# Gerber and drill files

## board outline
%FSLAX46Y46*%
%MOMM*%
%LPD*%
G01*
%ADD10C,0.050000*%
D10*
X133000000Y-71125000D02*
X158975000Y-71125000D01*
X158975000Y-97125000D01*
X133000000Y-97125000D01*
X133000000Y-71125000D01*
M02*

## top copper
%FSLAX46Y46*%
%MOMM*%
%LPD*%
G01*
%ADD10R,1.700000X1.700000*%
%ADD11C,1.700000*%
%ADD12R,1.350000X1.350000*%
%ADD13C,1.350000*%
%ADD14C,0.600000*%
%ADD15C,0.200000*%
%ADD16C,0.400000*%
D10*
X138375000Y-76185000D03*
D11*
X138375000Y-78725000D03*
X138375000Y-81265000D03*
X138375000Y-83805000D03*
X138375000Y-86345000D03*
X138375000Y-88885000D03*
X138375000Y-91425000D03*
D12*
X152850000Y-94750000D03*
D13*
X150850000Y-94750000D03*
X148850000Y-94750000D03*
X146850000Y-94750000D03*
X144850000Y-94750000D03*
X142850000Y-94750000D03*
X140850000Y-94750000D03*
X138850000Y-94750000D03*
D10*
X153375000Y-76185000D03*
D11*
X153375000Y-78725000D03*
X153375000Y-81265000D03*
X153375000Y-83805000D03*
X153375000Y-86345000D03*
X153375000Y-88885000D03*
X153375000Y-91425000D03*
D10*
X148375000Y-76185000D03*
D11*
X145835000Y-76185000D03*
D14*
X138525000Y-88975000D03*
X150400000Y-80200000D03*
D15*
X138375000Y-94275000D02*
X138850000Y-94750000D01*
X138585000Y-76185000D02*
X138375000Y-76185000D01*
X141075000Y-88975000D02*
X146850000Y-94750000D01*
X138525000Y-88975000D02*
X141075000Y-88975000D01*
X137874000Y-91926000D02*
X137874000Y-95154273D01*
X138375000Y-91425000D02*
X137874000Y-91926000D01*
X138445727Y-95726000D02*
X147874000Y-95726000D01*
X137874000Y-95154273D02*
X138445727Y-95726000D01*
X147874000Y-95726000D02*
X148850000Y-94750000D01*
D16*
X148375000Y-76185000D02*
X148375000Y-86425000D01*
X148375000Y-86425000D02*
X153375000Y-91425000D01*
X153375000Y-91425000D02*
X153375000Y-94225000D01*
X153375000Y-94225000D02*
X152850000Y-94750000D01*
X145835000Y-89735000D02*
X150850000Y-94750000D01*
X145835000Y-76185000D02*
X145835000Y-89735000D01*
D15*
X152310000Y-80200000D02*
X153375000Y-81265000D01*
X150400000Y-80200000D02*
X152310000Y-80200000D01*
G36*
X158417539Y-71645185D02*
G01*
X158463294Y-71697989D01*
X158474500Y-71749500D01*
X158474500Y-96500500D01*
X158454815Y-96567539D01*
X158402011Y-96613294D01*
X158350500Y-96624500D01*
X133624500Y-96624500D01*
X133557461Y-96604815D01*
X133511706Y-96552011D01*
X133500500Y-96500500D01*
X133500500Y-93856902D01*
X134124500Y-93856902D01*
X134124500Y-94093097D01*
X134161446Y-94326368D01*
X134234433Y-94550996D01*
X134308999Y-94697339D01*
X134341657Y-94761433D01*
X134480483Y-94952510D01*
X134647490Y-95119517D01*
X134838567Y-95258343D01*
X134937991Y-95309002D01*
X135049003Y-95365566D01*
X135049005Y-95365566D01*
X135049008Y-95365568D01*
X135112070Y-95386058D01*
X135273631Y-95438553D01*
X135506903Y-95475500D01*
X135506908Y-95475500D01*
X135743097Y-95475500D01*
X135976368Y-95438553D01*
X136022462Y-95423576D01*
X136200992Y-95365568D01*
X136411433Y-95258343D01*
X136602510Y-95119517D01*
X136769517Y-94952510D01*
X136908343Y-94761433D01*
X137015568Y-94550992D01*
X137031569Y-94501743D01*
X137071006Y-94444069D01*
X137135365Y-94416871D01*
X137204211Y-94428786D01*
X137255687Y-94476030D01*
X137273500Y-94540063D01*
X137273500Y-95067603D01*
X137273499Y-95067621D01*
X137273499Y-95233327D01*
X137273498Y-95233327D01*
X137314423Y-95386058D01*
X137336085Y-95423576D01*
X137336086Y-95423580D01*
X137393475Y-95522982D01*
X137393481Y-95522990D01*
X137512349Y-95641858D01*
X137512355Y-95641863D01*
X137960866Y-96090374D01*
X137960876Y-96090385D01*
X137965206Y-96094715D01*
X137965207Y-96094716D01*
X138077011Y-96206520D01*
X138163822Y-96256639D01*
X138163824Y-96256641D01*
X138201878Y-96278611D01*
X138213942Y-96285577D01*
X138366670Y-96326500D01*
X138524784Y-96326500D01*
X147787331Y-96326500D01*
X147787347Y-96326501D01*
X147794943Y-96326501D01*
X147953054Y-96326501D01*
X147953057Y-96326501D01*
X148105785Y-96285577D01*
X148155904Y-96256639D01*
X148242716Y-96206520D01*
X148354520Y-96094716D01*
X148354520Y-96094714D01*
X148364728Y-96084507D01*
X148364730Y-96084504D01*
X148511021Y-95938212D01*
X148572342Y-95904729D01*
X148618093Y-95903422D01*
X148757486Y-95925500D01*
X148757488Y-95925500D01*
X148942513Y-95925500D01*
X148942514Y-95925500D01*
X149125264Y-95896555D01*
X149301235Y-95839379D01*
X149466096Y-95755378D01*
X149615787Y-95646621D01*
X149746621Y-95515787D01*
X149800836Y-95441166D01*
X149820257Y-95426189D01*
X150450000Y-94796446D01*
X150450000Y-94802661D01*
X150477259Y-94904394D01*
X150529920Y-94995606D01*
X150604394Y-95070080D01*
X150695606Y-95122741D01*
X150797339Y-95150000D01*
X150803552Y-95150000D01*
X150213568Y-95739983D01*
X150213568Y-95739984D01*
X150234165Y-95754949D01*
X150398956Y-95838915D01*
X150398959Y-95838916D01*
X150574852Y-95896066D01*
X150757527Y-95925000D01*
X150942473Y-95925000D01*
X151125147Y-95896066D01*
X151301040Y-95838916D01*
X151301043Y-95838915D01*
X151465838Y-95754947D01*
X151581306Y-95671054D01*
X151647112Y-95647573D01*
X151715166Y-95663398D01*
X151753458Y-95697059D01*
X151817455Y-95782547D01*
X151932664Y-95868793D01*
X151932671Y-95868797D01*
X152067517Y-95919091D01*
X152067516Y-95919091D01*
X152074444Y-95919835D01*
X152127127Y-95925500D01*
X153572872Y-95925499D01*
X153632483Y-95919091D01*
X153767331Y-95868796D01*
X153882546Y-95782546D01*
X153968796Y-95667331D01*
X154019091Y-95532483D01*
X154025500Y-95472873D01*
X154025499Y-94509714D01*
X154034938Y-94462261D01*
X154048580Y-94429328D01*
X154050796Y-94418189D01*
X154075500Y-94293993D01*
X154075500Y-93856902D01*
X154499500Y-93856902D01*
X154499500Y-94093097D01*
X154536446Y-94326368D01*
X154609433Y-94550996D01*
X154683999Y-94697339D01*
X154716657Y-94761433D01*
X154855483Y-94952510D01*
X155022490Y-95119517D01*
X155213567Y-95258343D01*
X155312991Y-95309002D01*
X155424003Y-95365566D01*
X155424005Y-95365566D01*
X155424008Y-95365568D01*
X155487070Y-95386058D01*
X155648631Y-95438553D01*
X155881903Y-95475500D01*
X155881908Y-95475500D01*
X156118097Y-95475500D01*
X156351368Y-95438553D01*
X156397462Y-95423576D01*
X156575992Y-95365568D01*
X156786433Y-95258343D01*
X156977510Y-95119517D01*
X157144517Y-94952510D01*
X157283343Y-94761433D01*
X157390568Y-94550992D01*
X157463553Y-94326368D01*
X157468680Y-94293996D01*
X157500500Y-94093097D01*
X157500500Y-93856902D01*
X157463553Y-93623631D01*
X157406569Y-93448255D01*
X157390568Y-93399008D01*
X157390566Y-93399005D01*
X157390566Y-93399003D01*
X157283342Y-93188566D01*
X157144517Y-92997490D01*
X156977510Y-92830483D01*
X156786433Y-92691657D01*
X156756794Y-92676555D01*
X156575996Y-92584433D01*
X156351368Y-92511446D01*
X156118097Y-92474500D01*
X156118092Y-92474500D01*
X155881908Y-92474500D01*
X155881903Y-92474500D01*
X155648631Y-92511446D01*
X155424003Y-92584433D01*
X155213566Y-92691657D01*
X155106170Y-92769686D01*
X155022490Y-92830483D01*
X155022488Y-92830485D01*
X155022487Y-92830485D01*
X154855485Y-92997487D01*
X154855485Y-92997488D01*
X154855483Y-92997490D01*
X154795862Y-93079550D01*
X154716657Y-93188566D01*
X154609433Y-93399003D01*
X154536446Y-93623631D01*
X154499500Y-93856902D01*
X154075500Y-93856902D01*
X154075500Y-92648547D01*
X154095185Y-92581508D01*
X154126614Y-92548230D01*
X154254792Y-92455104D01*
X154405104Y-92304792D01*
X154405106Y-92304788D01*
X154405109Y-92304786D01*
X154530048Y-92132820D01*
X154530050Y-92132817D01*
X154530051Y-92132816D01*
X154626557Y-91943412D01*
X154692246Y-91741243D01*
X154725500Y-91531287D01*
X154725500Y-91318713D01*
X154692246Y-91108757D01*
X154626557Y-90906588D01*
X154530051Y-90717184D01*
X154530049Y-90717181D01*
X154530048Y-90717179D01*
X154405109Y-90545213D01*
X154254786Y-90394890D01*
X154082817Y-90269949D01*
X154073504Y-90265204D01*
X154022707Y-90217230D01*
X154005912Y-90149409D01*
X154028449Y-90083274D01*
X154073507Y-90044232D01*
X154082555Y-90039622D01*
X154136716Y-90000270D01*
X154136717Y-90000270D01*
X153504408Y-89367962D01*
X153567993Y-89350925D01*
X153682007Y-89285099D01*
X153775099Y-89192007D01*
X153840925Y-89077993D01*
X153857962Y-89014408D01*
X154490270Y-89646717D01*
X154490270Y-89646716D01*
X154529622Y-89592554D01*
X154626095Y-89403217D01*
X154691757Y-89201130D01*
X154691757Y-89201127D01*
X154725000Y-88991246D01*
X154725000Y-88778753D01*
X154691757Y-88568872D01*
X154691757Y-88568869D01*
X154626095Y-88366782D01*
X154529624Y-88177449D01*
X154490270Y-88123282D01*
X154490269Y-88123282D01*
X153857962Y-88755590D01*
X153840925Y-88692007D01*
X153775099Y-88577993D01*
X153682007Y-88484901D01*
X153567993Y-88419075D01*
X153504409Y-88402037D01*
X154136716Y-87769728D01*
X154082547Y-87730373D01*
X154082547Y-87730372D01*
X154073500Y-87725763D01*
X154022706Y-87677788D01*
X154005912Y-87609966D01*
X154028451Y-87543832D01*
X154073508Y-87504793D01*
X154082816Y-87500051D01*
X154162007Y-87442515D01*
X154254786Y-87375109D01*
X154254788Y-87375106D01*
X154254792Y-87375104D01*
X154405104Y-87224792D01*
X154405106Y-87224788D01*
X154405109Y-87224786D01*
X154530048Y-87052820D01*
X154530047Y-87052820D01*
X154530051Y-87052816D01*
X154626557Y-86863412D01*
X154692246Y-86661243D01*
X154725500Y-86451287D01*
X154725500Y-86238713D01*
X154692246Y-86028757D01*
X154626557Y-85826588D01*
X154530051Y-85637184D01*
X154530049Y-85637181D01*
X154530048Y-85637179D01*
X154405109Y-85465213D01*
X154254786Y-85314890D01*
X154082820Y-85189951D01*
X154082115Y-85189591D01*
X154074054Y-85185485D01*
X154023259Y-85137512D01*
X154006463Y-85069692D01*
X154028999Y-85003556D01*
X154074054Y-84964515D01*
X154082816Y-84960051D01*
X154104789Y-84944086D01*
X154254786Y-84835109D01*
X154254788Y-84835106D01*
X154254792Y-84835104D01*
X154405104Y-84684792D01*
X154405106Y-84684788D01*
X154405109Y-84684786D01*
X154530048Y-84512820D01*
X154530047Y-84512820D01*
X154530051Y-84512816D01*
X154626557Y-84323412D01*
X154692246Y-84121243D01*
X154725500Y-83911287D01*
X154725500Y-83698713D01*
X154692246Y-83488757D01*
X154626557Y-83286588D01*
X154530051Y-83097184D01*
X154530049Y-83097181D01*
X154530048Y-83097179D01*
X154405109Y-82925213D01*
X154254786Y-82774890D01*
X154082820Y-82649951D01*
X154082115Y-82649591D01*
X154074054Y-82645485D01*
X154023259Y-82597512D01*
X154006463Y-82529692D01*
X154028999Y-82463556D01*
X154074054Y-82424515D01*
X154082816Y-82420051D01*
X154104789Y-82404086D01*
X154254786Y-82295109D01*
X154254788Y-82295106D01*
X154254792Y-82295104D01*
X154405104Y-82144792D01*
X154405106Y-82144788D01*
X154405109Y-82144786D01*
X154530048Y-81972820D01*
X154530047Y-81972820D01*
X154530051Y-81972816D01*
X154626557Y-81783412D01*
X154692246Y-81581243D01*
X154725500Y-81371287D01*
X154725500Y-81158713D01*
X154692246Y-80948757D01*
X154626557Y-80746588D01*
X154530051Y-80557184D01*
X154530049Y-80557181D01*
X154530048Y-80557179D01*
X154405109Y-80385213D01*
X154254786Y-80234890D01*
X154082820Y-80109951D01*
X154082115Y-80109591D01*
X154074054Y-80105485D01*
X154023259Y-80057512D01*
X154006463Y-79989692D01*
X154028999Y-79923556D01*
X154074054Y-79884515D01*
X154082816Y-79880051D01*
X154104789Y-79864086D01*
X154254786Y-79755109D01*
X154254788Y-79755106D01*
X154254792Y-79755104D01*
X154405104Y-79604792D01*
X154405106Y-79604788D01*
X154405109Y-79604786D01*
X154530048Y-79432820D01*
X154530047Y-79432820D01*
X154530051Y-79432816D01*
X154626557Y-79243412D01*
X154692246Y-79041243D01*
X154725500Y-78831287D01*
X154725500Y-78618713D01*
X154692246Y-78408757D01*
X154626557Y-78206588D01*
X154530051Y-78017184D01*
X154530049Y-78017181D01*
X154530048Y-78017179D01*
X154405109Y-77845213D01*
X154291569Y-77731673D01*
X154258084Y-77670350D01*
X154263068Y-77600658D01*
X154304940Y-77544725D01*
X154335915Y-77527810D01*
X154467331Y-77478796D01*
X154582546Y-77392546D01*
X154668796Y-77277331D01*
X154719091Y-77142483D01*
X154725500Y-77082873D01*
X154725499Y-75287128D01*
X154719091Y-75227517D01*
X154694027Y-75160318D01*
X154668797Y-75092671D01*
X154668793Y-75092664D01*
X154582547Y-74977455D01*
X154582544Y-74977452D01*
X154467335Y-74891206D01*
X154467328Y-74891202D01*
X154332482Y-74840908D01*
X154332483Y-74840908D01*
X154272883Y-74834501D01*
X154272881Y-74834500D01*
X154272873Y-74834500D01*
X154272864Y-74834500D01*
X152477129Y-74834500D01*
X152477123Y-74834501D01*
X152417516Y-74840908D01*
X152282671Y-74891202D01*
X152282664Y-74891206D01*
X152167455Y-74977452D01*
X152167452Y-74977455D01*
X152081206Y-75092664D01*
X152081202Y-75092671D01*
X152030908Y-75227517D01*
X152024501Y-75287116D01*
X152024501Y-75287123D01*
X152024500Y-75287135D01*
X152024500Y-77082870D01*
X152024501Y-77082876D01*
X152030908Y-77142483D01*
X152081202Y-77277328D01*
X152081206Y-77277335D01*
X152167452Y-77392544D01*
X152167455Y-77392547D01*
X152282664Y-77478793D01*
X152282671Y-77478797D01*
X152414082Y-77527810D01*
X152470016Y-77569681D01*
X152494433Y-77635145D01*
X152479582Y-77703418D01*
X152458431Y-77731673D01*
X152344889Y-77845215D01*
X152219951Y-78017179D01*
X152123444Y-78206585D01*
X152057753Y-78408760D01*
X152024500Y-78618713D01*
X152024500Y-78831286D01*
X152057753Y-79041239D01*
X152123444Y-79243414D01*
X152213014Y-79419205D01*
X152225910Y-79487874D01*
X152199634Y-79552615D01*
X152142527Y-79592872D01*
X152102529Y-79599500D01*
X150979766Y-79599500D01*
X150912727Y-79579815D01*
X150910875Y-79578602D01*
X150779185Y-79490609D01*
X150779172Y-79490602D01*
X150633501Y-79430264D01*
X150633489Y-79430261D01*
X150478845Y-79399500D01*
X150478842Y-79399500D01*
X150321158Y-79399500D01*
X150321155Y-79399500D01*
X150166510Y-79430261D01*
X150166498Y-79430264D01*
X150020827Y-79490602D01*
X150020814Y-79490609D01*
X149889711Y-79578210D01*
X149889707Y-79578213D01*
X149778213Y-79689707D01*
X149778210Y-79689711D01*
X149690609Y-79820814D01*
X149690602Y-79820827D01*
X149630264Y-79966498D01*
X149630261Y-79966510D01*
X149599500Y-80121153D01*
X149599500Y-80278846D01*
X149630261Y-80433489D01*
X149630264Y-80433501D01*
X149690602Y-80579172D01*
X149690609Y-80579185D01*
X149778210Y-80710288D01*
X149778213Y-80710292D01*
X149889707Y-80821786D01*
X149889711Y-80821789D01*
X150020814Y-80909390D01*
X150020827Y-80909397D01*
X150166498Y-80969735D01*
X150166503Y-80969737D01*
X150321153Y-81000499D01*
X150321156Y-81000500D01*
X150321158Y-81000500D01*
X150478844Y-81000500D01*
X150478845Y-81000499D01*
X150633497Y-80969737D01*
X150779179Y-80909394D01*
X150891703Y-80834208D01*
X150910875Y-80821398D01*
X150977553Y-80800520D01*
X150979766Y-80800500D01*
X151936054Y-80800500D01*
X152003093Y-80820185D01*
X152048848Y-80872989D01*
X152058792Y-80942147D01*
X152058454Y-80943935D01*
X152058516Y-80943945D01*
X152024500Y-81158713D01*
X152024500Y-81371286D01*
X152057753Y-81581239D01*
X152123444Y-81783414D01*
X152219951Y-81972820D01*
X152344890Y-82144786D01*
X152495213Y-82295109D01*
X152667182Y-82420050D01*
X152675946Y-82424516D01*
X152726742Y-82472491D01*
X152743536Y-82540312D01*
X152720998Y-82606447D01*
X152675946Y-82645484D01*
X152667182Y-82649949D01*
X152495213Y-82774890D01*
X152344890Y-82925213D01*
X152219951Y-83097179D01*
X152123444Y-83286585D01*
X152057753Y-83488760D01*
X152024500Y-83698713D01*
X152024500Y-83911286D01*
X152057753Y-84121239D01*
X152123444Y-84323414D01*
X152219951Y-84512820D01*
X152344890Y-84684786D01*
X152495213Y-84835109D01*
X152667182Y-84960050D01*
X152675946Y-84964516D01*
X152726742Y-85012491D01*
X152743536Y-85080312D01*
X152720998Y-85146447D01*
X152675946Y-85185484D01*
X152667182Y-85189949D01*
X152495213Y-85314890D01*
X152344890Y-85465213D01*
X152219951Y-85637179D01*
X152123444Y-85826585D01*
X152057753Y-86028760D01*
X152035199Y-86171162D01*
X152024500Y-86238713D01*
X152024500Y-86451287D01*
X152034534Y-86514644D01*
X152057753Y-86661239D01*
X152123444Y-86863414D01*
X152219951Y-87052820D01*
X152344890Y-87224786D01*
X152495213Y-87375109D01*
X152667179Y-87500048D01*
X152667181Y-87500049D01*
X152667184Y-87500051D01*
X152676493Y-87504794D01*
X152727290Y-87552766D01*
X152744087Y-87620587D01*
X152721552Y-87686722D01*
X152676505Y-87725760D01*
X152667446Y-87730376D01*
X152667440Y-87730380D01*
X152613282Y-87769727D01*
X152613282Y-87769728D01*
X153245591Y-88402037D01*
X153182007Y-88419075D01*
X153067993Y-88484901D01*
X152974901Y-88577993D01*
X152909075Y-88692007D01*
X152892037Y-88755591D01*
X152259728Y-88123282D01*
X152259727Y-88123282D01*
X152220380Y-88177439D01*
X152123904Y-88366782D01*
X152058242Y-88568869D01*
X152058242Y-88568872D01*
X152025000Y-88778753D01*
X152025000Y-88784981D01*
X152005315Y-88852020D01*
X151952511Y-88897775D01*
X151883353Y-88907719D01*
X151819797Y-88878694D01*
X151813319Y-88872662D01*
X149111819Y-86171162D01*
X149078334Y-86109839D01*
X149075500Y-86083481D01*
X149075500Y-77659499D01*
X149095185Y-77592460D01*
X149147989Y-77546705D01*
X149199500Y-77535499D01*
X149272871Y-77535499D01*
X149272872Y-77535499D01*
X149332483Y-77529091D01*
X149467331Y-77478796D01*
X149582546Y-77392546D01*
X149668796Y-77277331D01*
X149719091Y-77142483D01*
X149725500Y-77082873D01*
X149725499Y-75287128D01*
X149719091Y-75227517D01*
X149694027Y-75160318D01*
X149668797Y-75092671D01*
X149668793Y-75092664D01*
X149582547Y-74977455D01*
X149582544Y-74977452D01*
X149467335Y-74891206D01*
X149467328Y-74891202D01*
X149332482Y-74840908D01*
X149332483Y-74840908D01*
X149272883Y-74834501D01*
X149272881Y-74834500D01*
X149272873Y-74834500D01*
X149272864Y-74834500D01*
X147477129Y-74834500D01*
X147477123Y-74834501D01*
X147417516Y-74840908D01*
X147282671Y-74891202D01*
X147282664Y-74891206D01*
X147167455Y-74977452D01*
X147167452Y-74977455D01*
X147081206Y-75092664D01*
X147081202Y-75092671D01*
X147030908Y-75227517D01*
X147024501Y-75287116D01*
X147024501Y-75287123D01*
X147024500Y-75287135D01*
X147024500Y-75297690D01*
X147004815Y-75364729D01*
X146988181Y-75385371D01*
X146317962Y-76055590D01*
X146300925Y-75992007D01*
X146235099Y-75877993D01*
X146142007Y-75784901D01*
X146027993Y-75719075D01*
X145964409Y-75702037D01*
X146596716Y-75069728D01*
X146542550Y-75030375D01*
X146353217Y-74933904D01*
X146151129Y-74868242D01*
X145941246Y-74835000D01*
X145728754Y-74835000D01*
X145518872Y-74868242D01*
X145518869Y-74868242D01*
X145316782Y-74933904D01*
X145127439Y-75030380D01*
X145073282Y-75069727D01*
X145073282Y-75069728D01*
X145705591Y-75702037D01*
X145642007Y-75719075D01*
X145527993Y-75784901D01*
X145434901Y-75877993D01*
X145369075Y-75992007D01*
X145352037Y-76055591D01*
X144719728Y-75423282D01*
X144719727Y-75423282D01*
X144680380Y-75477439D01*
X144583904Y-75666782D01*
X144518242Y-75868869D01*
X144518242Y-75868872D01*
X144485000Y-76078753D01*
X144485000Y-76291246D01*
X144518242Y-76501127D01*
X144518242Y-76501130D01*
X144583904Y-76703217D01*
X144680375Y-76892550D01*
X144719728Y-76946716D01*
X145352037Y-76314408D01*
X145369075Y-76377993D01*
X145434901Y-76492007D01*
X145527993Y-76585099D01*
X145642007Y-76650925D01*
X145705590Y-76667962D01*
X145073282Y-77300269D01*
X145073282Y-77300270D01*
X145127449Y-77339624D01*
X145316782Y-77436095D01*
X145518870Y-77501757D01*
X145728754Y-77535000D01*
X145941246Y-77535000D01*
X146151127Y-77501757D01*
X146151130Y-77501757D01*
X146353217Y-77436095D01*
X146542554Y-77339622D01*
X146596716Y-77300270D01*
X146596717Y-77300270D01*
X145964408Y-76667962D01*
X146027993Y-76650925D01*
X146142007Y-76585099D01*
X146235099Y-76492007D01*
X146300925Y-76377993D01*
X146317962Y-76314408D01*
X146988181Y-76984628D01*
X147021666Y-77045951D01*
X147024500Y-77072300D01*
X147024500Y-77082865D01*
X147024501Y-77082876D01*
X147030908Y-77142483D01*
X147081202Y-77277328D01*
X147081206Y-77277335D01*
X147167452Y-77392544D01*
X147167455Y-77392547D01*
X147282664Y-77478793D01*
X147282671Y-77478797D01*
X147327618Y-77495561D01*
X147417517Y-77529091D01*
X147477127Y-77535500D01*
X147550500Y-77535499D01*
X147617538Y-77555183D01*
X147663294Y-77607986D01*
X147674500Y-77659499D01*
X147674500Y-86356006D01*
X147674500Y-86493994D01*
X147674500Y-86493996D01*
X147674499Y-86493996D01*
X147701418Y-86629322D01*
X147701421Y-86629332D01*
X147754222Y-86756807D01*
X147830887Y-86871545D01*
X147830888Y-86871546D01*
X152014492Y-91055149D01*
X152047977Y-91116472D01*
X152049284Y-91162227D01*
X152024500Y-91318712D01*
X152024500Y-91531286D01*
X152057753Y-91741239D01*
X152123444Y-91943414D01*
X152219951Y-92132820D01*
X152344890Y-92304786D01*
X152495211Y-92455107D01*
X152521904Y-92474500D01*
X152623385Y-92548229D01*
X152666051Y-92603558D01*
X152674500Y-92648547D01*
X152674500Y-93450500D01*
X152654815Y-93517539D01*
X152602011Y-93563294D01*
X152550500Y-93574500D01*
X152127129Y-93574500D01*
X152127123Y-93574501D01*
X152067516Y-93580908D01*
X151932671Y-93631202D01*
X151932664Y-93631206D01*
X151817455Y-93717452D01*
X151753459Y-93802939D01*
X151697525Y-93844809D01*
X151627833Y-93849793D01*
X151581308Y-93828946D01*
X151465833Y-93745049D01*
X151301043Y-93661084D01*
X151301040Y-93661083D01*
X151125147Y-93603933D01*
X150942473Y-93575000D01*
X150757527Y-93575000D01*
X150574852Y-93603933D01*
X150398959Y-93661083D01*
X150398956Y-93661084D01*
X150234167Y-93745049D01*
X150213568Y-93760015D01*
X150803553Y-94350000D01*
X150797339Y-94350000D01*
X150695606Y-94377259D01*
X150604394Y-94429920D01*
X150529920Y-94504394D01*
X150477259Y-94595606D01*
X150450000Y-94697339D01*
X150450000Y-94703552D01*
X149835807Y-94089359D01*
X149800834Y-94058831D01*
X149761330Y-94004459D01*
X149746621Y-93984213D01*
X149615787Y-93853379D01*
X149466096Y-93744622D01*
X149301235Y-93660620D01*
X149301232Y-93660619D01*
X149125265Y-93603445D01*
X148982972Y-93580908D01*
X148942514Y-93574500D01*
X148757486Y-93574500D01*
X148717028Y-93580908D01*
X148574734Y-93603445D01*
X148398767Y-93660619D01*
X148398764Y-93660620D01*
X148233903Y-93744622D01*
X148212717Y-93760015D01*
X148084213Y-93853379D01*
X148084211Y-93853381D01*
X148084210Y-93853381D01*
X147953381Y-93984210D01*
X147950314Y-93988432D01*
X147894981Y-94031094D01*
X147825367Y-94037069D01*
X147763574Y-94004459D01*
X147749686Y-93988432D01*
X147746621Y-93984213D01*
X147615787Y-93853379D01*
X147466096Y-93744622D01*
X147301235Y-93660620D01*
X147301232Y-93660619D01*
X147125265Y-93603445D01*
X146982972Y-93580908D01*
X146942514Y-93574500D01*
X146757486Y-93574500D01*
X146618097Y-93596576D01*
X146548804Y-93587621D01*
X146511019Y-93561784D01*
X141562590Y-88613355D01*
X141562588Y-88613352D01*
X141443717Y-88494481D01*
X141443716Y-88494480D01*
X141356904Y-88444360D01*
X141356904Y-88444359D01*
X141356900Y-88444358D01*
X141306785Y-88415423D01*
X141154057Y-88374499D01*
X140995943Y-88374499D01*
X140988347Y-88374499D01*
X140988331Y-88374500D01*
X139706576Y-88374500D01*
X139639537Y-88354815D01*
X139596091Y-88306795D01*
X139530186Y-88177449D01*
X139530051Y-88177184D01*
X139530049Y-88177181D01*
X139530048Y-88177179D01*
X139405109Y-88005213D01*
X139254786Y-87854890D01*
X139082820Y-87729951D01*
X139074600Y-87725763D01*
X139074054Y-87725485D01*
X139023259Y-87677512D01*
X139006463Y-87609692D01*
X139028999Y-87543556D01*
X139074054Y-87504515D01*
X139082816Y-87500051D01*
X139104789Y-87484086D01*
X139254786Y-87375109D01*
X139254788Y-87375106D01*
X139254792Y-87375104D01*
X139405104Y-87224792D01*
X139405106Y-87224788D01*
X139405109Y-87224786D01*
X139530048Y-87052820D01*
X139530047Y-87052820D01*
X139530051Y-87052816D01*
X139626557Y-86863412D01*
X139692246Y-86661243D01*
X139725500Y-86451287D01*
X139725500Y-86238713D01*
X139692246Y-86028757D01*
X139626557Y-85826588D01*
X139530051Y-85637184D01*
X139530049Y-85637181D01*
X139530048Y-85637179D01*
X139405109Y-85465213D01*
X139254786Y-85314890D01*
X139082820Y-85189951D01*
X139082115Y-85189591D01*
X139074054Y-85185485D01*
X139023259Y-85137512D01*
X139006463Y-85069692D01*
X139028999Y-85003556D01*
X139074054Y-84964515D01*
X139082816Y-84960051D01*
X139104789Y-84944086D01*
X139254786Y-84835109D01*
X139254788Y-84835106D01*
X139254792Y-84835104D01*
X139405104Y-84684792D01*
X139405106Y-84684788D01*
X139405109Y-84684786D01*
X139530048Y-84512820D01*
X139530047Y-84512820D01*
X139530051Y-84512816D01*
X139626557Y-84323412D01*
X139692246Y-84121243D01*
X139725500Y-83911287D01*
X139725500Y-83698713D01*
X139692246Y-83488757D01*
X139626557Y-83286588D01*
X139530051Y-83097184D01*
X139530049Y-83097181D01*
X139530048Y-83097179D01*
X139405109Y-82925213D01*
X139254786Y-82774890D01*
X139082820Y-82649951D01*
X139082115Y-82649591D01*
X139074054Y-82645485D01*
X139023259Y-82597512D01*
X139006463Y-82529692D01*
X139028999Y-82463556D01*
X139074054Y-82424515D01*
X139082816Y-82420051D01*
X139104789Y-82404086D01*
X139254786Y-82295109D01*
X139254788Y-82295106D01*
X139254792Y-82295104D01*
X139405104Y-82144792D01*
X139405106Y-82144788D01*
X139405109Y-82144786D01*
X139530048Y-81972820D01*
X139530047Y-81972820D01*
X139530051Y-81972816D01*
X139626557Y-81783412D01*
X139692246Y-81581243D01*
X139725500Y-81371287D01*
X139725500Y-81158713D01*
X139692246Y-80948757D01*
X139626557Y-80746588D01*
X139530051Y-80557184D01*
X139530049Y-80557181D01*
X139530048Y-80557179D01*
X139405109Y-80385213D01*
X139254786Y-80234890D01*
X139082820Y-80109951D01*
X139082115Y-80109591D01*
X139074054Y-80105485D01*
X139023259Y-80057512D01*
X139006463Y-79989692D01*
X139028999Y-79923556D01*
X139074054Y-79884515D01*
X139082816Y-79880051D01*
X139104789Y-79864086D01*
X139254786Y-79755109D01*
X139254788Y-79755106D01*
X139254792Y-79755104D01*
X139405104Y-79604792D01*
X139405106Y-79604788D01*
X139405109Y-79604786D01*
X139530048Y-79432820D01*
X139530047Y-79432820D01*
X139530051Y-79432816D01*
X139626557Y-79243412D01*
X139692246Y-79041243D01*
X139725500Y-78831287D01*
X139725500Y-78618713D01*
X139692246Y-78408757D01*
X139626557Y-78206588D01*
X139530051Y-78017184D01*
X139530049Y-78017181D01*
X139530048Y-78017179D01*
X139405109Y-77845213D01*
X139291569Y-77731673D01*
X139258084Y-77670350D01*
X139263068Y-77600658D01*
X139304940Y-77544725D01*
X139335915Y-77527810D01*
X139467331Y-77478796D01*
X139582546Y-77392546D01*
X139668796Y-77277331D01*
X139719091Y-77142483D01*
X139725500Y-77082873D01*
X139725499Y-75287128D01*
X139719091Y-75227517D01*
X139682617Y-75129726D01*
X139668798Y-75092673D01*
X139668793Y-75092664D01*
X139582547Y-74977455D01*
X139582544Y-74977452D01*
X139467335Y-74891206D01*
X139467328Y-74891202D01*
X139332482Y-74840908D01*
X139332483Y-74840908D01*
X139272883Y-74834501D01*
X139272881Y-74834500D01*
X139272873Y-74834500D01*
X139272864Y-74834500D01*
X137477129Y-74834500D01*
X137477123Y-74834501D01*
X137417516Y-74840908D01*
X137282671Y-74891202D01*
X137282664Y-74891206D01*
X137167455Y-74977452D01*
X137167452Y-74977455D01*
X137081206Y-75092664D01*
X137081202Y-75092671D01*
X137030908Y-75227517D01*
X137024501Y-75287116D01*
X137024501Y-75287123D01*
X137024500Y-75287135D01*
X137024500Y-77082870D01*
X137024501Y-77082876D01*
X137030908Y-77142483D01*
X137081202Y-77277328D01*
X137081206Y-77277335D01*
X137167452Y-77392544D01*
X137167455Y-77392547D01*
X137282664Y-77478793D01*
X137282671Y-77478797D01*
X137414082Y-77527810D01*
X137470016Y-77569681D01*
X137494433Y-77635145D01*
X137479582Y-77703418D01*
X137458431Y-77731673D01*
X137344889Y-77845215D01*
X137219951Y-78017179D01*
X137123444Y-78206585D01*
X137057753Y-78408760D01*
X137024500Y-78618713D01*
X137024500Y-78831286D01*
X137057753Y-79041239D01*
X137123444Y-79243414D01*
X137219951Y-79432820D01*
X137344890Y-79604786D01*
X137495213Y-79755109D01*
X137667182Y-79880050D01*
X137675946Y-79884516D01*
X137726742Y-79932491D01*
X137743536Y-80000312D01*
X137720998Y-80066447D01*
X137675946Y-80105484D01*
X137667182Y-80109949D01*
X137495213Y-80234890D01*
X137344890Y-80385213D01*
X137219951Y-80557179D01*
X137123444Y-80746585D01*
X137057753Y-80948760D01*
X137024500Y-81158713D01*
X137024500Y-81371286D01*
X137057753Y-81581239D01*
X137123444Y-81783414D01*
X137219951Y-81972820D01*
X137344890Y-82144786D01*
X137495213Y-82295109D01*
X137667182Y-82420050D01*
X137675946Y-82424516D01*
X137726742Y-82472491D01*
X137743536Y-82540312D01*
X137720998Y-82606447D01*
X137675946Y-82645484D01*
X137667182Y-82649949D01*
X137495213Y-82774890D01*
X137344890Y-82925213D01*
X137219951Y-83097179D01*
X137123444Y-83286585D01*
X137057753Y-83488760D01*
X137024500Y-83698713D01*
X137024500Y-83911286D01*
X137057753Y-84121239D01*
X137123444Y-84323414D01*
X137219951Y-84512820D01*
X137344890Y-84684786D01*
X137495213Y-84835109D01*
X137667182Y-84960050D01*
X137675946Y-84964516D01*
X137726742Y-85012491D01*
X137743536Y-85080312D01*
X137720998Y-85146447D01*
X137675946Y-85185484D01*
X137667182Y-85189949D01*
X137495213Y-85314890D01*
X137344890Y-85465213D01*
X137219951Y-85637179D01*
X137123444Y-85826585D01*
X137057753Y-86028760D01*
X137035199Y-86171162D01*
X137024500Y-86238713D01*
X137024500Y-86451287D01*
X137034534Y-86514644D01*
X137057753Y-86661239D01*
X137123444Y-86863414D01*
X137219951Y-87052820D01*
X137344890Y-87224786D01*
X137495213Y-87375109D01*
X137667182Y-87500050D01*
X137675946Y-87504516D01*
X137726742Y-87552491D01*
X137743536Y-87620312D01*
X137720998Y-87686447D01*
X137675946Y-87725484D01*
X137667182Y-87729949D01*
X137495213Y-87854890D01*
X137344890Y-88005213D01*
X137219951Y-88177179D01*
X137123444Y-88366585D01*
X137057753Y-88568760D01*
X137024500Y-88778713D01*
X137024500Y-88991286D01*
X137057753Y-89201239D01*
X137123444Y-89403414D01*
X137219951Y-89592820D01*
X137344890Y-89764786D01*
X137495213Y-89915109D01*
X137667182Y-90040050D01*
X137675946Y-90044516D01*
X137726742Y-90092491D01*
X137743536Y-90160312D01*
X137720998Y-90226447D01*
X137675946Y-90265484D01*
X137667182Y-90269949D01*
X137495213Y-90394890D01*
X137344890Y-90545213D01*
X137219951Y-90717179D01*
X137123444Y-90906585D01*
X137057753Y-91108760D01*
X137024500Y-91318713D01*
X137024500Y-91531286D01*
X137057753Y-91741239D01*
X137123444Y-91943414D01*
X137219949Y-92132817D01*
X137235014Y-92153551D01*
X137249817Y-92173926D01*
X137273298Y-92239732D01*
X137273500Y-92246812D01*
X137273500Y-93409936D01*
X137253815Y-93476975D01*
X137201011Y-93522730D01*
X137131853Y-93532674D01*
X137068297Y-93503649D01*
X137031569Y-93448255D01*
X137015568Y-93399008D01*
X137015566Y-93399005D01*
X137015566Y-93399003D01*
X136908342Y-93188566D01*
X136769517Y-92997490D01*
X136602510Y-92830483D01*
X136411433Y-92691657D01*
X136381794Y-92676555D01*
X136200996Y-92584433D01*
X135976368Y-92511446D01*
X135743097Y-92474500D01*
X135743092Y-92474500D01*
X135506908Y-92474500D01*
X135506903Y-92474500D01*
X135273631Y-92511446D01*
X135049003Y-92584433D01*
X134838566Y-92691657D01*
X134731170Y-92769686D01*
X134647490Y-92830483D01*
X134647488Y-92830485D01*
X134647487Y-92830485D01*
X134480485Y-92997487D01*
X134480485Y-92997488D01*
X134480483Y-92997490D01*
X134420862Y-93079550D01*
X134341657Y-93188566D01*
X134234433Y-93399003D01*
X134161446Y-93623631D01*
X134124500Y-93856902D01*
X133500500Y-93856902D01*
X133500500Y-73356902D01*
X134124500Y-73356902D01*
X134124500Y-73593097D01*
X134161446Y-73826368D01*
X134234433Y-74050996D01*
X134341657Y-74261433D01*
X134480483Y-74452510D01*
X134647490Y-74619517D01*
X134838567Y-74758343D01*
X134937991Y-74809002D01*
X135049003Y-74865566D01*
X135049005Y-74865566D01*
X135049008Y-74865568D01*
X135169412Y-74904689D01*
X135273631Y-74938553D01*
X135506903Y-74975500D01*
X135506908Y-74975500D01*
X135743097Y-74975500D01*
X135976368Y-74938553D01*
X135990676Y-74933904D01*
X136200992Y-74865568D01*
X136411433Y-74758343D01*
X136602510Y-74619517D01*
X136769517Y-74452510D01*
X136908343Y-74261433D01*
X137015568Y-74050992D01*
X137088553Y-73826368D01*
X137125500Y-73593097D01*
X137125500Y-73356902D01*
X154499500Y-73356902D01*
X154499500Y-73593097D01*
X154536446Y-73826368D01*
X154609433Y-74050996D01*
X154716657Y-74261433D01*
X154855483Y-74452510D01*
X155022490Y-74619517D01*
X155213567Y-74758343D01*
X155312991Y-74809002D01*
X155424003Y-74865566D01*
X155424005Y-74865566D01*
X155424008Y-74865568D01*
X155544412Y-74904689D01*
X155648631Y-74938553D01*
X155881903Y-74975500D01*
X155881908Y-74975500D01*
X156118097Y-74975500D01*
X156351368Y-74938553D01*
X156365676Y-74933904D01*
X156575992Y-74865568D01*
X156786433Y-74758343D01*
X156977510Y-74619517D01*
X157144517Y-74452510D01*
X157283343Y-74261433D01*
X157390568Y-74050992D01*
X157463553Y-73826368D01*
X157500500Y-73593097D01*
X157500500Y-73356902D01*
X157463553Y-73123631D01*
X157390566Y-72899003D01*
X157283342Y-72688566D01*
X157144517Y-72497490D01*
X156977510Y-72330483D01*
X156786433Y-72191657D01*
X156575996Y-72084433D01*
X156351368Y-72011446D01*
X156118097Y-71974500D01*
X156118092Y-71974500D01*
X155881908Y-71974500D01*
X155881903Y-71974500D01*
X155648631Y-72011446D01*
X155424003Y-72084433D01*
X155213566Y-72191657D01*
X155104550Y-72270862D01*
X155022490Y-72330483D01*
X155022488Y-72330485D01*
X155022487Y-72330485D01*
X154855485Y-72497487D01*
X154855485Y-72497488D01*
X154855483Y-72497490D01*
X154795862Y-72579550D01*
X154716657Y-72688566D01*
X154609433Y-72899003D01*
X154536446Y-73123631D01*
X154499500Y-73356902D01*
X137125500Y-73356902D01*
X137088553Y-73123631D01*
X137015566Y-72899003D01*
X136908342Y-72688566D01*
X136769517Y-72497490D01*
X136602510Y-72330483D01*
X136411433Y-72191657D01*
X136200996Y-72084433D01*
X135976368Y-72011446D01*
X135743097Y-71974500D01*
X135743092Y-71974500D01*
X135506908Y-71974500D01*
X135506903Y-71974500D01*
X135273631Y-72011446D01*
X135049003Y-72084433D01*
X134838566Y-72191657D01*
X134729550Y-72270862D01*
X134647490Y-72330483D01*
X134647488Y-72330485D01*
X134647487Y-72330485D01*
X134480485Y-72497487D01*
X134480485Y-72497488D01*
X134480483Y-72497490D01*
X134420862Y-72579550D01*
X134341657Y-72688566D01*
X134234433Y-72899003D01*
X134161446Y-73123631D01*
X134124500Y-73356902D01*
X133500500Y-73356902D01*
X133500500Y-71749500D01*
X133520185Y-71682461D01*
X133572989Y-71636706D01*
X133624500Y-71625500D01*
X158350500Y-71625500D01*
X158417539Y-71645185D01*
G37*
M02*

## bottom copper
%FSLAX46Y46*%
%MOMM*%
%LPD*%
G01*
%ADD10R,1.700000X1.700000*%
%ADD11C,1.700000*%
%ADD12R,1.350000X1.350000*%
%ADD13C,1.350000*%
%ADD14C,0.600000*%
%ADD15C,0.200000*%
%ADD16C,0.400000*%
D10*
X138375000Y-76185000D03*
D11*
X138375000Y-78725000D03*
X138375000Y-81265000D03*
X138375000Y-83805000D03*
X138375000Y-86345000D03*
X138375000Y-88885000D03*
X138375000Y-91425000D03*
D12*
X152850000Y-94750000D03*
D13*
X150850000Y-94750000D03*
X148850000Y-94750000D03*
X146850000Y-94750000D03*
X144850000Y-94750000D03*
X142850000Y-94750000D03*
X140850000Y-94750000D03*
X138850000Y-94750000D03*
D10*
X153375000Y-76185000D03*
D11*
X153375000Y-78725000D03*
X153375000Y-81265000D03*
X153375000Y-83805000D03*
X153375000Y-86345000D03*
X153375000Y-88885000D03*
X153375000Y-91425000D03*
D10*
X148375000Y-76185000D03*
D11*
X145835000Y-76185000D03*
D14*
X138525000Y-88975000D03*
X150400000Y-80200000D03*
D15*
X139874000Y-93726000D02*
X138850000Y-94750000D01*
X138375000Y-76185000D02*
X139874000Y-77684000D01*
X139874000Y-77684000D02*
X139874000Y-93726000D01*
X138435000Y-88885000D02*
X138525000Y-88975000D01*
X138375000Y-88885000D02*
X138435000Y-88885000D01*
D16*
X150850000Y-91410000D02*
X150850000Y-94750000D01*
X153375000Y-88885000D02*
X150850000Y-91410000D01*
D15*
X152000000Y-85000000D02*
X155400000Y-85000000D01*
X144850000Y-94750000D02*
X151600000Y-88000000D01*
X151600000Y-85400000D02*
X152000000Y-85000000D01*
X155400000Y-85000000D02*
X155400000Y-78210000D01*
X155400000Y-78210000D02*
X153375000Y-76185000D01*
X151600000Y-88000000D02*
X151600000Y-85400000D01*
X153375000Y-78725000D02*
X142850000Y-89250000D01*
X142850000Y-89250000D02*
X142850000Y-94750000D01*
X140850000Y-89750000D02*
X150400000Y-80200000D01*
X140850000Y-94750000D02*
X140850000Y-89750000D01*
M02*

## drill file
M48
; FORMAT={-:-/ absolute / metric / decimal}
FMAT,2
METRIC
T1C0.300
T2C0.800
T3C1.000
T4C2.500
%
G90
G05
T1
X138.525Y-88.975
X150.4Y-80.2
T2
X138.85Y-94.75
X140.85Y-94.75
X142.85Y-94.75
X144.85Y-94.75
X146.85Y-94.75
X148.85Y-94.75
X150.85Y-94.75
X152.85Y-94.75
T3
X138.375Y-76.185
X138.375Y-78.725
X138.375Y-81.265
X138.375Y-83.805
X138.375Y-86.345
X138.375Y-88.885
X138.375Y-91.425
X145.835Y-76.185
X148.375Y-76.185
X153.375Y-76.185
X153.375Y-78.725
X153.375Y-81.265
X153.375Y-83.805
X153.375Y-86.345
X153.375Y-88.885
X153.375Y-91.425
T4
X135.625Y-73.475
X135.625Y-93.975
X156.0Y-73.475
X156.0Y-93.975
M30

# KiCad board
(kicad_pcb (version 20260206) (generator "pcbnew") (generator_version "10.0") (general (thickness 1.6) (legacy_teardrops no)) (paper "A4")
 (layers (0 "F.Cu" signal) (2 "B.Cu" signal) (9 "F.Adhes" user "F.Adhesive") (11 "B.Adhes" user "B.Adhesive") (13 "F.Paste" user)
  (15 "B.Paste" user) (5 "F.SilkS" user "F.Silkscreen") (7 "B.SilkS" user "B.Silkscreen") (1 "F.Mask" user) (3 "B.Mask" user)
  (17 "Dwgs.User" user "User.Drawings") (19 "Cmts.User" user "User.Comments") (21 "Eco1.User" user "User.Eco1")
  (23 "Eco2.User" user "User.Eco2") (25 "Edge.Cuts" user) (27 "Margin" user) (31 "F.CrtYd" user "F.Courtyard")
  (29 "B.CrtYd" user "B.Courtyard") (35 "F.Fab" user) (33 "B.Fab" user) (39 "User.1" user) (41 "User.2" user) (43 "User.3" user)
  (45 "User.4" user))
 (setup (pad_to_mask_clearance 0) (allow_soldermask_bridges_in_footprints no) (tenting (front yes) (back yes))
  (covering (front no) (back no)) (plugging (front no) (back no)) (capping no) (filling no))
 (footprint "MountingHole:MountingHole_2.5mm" (layer "F.Cu") (at 135.625 73.475)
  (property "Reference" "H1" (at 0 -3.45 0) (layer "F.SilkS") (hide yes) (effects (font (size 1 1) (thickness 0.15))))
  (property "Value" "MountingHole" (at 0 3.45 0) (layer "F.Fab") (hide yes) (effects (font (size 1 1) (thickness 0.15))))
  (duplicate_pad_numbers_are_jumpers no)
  (pad "" np_thru_hole circle (at 0 0) (size 2.5 2.5) (drill 2.5) (layers "*.Cu" "*.Mask")))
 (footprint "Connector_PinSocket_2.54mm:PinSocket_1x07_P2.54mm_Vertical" (layer "F.Cu") (at 138.375 76.185)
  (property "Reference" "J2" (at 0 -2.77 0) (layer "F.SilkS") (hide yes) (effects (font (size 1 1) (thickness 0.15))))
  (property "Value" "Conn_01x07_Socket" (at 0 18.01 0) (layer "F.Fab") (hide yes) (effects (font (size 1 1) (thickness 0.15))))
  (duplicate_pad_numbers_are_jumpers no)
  (pad "1" thru_hole rect (at 0 0) (size 1.7 1.7) (drill 1) (layers "*.Cu" "*.Mask") (remove_unused_layers no) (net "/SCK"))
  (pad "2" thru_hole circle (at 0 2.54) (size 1.7 1.7) (drill 1) (layers "*.Cu" "*.Mask") (remove_unused_layers no)
   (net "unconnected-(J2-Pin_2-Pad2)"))
  (pad "3" thru_hole circle (at 0 5.08) (size 1.7 1.7) (drill 1) (layers "*.Cu" "*.Mask") (remove_unused_layers no)
   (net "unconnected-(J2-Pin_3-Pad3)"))
  (pad "4" thru_hole circle (at 0 7.62) (size 1.7 1.7) (drill 1) (layers "*.Cu" "*.Mask") (remove_unused_layers no)
   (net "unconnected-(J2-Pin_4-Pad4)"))
  (pad "5" thru_hole circle (at 0 10.16) (size 1.7 1.7) (drill 1) (layers "*.Cu" "*.Mask") (remove_unused_layers no)
   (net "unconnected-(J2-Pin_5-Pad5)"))
  (pad "6" thru_hole circle (at 0 12.7) (size 1.7 1.7) (drill 1) (layers "*.Cu" "*.Mask") (remove_unused_layers no) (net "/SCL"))
  (pad "7" thru_hole circle (at 0 15.24) (size 1.7 1.7) (drill 1) (layers "*.Cu" "*.Mask") (remove_unused_layers no) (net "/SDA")))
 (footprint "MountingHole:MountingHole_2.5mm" (layer "F.Cu") (at 156.125 93.975)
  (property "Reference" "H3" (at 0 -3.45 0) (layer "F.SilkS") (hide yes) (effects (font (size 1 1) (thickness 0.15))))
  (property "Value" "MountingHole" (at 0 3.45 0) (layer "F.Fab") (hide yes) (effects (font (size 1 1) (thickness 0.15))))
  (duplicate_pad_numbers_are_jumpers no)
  (pad "" np_thru_hole circle (at -0.125 0) (size 2.5 2.5) (drill 2.5) (layers "*.Cu" "*.Mask")))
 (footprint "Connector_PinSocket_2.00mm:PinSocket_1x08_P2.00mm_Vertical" (layer "F.Cu") (at 152.85 94.75 -90)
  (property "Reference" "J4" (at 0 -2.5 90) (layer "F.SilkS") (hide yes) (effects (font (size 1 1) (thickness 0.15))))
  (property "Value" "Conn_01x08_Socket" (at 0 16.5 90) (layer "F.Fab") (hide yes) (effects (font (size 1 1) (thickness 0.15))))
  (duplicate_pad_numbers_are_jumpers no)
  (pad "1" thru_hole rect (at 0 0 270) (size 1.35 1.35) (drill 0.8) (layers "*.Cu" "*.Mask") (remove_unused_layers no) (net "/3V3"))
  (pad "2" thru_hole circle (at 0 2 270) (size 1.35 1.35) (drill 0.8) (layers "*.Cu" "*.Mask") (remove_unused_layers no) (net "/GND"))
  (pad "3" thru_hole circle (at 0 4 270) (size 1.35 1.35) (drill 0.8) (layers "*.Cu" "*.Mask") (remove_unused_layers no) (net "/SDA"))
  (pad "4" thru_hole circle (at 0 6 270) (size 1.35 1.35) (drill 0.8) (layers "*.Cu" "*.Mask") (remove_unused_layers no) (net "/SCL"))
  (pad "5" thru_hole circle (at 0 8 270) (size 1.35 1.35) (drill 0.8) (layers "*.Cu" "*.Mask") (remove_unused_layers no) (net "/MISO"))
  (pad "6" thru_hole circle (at 0 10 270) (size 1.35 1.35) (drill 0.8) (layers "*.Cu" "*.Mask") (remove_unused_layers no) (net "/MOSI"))
  (pad "7" thru_hole circle (at 0 12 270) (size 1.35 1.35) (drill 0.8) (layers "*.Cu" "*.Mask") (remove_unused_layers no) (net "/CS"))
  (pad "8" thru_hole circle (at 0 14 270) (size 1.35 1.35) (drill 0.8) (layers "*.Cu" "*.Mask") (remove_unused_layers no) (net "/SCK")))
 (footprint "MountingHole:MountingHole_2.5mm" (layer "F.Cu") (at 156.125 73.475)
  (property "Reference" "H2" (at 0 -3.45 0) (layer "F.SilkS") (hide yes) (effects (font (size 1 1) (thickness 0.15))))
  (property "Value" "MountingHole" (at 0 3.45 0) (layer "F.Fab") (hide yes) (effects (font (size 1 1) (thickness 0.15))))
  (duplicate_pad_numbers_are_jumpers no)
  (pad "" np_thru_hole circle (at -0.125 0) (size 2.5 2.5) (drill 2.5) (layers "*.Cu" "*.Mask")))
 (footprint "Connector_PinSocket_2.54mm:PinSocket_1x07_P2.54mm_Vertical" (layer "F.Cu") (at 153.375 76.185)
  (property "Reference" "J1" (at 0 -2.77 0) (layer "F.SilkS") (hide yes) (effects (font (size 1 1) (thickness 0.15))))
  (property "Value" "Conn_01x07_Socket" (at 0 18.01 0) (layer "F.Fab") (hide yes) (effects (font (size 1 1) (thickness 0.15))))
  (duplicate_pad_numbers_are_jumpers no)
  (pad "1" thru_hole rect (at 0 0) (size 1.7 1.7) (drill 1) (layers "*.Cu" "*.Mask") (remove_unused_layers no) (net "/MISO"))
  (pad "2" thru_hole circle (at 0 2.54) (size 1.7 1.7) (drill 1) (layers "*.Cu" "*.Mask") (remove_unused_layers no) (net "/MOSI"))
  (pad "3" thru_hole circle (at 0 5.08) (size 1.7 1.7) (drill 1) (layers "*.Cu" "*.Mask") (remove_unused_layers no) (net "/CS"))
  (pad "4" thru_hole circle (at 0 7.62) (size 1.7 1.7) (drill 1) (layers "*.Cu" "*.Mask") (remove_unused_layers no)
   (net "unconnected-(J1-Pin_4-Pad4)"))
  (pad "5" thru_hole circle (at 0 10.16) (size 1.7 1.7) (drill 1) (layers "*.Cu" "*.Mask") (remove_unused_layers no)
   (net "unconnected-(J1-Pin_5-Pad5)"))
  (pad "6" thru_hole circle (at 0 12.7) (size 1.7 1.7) (drill 1) (layers "*.Cu" "*.Mask") (remove_unused_layers no) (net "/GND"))
  (pad "7" thru_hole circle (at 0 15.24) (size 1.7 1.7) (drill 1) (layers "*.Cu" "*.Mask") (remove_unused_layers no) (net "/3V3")))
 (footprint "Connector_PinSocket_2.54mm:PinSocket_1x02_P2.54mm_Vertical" (layer "F.Cu") (at 148.375 76.185 -90)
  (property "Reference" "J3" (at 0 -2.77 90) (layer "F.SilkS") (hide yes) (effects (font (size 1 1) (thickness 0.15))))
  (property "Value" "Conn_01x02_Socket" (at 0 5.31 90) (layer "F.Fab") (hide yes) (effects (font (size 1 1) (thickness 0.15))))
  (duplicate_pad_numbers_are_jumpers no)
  (pad "1" thru_hole rect (at 0 0 270) (size 1.7 1.7) (drill 1) (layers "*.Cu" "*.Mask") (remove_unused_layers no) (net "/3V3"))
  (pad "2" thru_hole circle (at 0 2.54 270) (size 1.7 1.7) (drill 1) (layers "*.Cu" "*.Mask") (remove_unused_layers no) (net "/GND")))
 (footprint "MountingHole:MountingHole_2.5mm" (layer "F.Cu") (at 135.625 93.975)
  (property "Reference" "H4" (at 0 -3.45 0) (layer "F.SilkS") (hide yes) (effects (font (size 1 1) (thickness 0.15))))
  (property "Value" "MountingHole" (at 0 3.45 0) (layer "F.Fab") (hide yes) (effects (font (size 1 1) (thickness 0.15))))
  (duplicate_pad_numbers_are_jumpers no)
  (pad "" np_thru_hole circle (at 0 0) (size 2.5 2.5) (drill 2.5) (layers "*.Cu" "*.Mask")))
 (gr_rect (start 133 71.125) (end 158.975 97.125) (stroke (width 0.05) (type default)) (fill no) (layer "Edge.Cuts"))
 (segment (start 138.375 94.275) (end 138.85 94.75) (width 0.2) (layer "F.Cu") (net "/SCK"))
 (segment (start 138.585 76.185) (end 138.375 76.185) (width 0.2) (layer "F.Cu") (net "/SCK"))
 (segment (start 139.874 93.726) (end 138.85 94.75) (width 0.2) (layer "B.Cu") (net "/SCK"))
 (segment (start 138.375 76.185) (end 139.874 77.684) (width 0.2) (layer "B.Cu") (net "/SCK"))
 (segment (start 139.874 77.684) (end 139.874 93.726) (width 0.2) (layer "B.Cu") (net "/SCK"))
 (segment (start 141.075 88.975) (end 146.85 94.75) (width 0.2) (layer "F.Cu") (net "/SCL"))
 (segment (start 138.525 88.975) (end 141.075 88.975) (width 0.2) (layer "F.Cu") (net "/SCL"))
 (via (at 138.525 88.975) (size 0.6) (drill 0.3) (layers "F.Cu" "B.Cu") (capping no) (covering (front no) (back no))
  (plugging (front no) (back no)) (filling no) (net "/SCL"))
 (segment (start 138.435 88.885) (end 138.525 88.975) (width 0.2) (layer "B.Cu") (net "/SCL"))
 (segment (start 138.375 88.885) (end 138.435 88.885) (width 0.2) (layer "B.Cu") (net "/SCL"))
 (segment (start 137.874 91.926) (end 137.874 95.154273) (width 0.2) (layer "F.Cu") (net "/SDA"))
 (segment (start 138.375 91.425) (end 137.874 91.926) (width 0.2) (layer "F.Cu") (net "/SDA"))
 (segment (start 138.445727 95.726) (end 147.874 95.726) (width 0.2) (layer "F.Cu") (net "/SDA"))
 (segment (start 137.874 95.154273) (end 138.445727 95.726) (width 0.2) (layer "F.Cu") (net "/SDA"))
 (segment (start 147.874 95.726) (end 148.85 94.75) (width 0.2) (layer "F.Cu") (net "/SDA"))
 (segment (start 148.375 76.185) (end 148.375 86.425) (width 0.4) (layer "F.Cu") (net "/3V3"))
 (segment (start 148.375 86.425) (end 153.375 91.425) (width 0.4) (layer "F.Cu") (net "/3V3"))
 (segment (start 153.375 91.425) (end 153.375 94.225) (width 0.4) (layer "F.Cu") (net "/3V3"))
 (segment (start 153.375 94.225) (end 152.85 94.75) (width 0.4) (layer "F.Cu") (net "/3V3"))
 (segment (start 145.835 89.735) (end 150.85 94.75) (width 0.4) (layer "F.Cu") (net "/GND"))
 (segment (start 145.835 76.185) (end 145.835 89.735) (width 0.4) (layer "F.Cu") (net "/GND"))
 (segment (start 150.85 91.41) (end 150.85 94.75) (width 0.4) (layer "B.Cu") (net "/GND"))
 (segment (start 153.375 88.885) (end 150.85 91.41) (width 0.4) (layer "B.Cu") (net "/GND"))
 (segment (start 152 85) (end 155.4 85) (width 0.2) (layer "B.Cu") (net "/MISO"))
 (segment (start 144.85 94.75) (end 151.6 88) (width 0.2) (layer "B.Cu") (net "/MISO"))
 (segment (start 151.6 85.4) (end 152 85) (width 0.2) (layer "B.Cu") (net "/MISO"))
 (segment (start 155.4 85) (end 155.4 78.21) (width 0.2) (layer "B.Cu") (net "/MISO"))
 (segment (start 155.4 78.21) (end 153.375 76.185) (width 0.2) (layer "B.Cu") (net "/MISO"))
 (segment (start 151.6 88) (end 151.6 85.4) (width 0.2) (layer "B.Cu") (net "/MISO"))
 (segment (start 153.375 78.725) (end 142.85 89.25) (width 0.2) (layer "B.Cu") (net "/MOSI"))
 (segment (start 142.85 89.25) (end 142.85 94.75) (width 0.2) (layer "B.Cu") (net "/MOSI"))
 (segment (start 152.31 80.2) (end 153.375 81.265) (width 0.2) (layer "F.Cu") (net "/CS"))
 (segment (start 150.4 80.2) (end 152.31 80.2) (width 0.2) (layer "F.Cu") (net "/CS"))
 (via (at 150.4 80.2) (size 0.6) (drill 0.3) (layers "F.Cu" "B.Cu") (capping no) (covering (front no) (back no))
  (plugging (front no) (back no)) (filling no) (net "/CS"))
 (segment (start 140.85 89.75) (end 150.4 80.2) (width 0.2) (layer "B.Cu") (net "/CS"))
 (segment (start 140.85 94.75) (end 140.85 89.75) (width 0.2) (layer "B.Cu") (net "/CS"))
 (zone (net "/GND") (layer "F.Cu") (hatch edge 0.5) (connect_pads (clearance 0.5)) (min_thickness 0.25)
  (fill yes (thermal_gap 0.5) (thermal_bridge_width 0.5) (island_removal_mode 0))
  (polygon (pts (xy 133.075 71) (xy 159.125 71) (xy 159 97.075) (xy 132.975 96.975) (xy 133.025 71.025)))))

